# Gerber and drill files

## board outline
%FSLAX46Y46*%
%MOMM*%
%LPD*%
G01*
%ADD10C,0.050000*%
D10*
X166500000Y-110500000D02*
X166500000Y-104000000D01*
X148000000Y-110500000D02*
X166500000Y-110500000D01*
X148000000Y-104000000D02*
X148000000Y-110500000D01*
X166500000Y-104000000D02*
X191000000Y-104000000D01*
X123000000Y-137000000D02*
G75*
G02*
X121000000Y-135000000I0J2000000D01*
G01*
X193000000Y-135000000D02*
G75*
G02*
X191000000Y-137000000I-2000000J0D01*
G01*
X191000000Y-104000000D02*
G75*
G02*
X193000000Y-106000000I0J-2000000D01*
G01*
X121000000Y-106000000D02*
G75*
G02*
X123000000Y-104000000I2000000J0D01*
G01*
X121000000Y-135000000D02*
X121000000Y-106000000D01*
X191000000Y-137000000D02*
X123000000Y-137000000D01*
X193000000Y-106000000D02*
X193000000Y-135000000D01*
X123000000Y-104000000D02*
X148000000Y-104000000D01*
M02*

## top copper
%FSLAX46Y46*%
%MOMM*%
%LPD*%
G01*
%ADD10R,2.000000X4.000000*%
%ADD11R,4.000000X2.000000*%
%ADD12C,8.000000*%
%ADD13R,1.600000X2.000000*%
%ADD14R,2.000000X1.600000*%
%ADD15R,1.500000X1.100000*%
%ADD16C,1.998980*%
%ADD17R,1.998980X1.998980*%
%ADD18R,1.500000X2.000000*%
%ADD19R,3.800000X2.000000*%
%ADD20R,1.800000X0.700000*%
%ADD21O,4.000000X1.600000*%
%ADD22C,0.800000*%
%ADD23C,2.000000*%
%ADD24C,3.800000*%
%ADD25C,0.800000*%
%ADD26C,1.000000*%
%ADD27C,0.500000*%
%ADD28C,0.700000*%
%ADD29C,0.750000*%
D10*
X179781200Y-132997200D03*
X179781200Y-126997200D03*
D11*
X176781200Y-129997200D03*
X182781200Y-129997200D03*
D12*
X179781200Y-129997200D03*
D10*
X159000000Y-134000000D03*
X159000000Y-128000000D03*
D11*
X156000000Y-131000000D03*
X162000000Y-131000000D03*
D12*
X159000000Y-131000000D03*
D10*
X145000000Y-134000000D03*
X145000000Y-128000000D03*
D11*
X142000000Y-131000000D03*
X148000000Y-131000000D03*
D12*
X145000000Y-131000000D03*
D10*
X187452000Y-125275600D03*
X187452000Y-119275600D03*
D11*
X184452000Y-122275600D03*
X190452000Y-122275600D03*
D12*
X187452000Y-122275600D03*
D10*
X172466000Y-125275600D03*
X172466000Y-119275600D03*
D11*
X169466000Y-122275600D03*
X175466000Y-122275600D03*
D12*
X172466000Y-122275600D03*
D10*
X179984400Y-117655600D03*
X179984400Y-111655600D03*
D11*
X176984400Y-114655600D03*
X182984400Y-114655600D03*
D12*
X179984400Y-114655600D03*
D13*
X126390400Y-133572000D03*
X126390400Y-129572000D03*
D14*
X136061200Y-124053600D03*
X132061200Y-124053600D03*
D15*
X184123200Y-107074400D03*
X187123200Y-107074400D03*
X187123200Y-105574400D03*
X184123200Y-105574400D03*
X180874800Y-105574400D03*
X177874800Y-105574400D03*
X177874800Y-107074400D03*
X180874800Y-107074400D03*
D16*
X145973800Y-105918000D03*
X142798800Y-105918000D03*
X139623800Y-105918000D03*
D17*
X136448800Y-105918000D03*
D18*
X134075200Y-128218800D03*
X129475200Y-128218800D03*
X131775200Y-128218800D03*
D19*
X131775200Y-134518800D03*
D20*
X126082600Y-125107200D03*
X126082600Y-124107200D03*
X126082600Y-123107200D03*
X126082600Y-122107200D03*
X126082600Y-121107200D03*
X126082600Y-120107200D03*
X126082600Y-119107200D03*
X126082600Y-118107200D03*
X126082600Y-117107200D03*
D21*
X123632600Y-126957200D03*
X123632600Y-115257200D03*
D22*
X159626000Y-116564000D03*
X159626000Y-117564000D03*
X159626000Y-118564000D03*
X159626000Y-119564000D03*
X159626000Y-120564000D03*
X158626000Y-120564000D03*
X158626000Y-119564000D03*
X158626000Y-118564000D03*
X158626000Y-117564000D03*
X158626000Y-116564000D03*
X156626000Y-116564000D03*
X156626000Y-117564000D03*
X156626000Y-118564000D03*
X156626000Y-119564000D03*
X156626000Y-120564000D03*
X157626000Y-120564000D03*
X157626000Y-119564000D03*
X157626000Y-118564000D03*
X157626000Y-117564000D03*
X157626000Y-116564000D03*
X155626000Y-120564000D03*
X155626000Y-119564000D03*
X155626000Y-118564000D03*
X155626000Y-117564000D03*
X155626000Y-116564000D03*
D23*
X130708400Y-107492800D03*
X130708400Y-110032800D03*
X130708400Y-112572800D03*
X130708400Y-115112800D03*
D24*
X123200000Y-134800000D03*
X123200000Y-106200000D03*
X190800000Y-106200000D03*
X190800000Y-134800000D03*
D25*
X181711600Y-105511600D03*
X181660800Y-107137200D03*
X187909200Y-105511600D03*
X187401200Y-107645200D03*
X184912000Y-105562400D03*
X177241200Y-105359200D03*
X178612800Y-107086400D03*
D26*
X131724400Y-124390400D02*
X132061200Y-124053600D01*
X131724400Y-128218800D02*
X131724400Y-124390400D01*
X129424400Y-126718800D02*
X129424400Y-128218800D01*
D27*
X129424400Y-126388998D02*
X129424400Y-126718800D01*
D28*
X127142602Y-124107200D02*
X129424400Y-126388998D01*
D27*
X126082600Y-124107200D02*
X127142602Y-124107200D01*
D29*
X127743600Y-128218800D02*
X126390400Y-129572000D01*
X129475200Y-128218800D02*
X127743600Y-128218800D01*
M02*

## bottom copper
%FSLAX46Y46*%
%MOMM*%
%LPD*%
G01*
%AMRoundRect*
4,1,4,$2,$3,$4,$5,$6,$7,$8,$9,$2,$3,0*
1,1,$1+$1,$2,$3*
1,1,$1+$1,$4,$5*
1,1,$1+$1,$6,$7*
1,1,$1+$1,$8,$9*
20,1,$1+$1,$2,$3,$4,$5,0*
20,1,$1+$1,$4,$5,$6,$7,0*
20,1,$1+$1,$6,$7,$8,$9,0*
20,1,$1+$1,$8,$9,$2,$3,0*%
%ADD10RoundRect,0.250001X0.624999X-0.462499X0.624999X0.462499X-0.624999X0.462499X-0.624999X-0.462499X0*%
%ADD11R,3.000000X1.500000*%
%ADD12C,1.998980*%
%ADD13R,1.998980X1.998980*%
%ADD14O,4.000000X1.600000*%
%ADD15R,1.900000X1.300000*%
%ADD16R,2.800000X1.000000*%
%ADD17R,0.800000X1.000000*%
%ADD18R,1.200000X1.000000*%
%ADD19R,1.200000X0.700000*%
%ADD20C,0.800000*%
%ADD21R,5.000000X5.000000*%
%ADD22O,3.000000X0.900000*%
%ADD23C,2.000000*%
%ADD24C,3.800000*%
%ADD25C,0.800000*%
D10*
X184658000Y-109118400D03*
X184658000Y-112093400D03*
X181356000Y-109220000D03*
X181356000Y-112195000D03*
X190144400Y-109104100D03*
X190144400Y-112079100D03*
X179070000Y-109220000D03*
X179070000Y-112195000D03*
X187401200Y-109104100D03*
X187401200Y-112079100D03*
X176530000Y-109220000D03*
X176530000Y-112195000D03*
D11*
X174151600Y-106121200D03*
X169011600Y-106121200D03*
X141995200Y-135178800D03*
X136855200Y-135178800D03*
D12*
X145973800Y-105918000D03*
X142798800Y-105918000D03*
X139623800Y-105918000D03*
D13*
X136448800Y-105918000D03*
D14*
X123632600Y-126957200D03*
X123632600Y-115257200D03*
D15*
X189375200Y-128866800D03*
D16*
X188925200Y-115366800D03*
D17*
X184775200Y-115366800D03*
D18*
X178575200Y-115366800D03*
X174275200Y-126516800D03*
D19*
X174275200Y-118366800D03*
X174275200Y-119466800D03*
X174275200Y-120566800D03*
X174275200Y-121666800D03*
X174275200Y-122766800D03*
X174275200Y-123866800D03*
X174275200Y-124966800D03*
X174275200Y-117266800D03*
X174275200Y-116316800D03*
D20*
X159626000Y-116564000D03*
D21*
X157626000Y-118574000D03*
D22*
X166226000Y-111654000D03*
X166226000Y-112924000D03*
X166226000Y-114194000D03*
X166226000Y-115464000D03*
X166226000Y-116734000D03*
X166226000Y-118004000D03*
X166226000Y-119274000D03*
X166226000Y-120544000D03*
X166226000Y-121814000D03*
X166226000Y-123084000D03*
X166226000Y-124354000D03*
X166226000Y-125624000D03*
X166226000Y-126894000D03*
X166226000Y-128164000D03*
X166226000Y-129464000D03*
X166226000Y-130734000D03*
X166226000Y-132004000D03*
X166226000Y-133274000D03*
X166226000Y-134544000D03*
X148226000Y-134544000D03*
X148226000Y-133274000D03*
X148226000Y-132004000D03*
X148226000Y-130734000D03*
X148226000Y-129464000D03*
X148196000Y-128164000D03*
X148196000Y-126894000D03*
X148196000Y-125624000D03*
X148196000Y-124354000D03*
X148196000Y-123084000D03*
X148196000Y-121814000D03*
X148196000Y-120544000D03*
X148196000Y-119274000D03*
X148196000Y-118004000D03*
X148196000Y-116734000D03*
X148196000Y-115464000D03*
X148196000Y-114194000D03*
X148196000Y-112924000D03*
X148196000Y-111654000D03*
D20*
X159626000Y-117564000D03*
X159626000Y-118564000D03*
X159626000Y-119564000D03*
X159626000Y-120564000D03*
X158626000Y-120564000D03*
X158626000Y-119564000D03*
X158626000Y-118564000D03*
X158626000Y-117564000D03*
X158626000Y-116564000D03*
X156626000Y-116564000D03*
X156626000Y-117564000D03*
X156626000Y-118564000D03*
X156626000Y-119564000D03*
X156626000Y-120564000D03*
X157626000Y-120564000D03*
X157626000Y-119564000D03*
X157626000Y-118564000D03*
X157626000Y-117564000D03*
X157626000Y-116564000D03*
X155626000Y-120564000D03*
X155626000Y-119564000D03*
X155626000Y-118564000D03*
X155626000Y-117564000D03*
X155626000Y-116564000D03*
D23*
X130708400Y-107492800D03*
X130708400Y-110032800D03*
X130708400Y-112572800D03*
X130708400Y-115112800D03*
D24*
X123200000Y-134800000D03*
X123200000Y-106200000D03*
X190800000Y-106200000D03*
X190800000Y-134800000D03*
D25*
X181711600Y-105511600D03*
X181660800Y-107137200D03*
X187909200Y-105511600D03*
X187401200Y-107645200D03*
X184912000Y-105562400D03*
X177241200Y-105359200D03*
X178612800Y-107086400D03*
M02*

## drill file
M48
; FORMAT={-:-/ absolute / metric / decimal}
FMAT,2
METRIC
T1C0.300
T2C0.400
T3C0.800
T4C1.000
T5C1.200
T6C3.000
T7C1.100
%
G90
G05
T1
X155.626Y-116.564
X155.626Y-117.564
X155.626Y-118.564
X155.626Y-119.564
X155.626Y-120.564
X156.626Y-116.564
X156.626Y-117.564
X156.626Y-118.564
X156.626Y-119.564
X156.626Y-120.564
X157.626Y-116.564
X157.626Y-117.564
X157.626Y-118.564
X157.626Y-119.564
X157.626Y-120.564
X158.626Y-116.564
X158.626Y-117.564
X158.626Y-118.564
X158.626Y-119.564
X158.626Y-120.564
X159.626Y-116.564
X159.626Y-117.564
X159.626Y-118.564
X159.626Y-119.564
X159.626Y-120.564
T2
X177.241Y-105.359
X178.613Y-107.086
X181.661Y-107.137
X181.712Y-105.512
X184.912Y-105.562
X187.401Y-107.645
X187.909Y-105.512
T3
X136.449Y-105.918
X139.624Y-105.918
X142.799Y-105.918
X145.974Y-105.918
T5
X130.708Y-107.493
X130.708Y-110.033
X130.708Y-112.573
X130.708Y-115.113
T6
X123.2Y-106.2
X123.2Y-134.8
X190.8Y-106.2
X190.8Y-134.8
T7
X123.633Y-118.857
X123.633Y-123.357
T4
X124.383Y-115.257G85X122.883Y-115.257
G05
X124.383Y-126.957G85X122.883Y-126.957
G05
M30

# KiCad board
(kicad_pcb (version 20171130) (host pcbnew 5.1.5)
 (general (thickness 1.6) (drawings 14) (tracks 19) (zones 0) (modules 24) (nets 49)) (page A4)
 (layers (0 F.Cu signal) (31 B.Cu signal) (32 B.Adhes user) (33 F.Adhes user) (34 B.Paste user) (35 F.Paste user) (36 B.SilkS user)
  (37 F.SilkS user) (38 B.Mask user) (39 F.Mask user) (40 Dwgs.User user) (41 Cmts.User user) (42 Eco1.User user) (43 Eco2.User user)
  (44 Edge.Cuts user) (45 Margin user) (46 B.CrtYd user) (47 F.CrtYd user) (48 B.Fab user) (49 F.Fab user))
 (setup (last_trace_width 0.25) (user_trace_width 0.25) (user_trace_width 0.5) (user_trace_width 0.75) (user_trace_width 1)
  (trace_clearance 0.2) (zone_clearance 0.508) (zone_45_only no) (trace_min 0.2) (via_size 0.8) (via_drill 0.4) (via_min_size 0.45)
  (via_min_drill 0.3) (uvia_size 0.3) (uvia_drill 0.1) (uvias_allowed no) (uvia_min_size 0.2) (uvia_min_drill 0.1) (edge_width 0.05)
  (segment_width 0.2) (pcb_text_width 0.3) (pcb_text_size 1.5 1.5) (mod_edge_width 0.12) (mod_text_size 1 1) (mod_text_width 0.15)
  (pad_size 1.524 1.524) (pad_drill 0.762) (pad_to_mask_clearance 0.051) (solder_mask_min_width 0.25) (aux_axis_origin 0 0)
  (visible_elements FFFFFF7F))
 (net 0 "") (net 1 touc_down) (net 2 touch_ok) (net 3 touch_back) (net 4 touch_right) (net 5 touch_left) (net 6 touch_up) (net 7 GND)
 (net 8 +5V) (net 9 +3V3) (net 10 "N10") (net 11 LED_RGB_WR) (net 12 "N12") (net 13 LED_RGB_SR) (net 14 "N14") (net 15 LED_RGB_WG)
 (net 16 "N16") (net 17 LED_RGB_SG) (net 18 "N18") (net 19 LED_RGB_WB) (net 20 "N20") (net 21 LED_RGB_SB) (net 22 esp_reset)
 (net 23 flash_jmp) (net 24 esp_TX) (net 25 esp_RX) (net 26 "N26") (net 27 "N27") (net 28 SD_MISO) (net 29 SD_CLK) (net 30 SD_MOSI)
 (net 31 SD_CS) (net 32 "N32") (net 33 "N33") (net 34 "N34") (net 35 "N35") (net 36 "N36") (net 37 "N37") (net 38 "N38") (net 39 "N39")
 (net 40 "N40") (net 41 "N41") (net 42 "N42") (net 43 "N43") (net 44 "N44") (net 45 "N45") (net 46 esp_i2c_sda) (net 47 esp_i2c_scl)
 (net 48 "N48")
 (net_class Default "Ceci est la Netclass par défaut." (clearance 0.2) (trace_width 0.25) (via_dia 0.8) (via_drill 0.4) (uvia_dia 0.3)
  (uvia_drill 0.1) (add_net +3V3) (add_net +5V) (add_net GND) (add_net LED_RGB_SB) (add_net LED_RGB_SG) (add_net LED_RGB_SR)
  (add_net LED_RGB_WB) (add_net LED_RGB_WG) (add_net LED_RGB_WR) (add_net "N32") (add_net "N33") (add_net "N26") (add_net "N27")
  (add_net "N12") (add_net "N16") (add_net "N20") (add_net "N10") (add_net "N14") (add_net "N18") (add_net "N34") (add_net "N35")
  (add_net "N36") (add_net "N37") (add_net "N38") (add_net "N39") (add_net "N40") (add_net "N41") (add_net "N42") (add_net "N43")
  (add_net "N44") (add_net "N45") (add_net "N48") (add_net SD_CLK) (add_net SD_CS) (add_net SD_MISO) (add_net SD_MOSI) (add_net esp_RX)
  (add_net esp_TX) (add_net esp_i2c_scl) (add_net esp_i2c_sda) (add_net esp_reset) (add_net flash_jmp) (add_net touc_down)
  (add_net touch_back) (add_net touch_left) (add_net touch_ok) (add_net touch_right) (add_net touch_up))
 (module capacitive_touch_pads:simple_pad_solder (layer F.Cu) (at 179.7812 129.9972)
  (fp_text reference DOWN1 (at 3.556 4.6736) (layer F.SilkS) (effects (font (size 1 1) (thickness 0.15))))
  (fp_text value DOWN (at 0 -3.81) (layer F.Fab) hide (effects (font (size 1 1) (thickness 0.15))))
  (pad 1 smd rect (at 0 3 180) (size 2 4) (layers F.Cu F.Paste F.Mask) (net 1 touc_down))
  (pad 1 smd rect (at 0 -3 180) (size 2 4) (layers F.Cu F.Paste F.Mask) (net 1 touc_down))
  (pad 1 smd rect (at -3 0 90) (size 2 4) (layers F.Cu F.Paste F.Mask) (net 1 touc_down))
  (pad 1 smd rect (at 3 0 90) (size 2 4) (layers F.Cu F.Paste F.Mask) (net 1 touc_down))
  (pad 1 smd circle (at 0 0) (size 8 8) (layers F.Cu F.Paste F.Mask) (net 1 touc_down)))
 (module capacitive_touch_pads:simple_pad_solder (layer F.Cu) (at 159 131)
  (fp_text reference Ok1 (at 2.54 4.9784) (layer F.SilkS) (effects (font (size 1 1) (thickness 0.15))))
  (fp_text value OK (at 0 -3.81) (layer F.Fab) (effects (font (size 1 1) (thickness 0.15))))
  (pad 1 smd rect (at 0 3 180) (size 2 4) (layers F.Cu F.Paste F.Mask) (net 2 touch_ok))
  (pad 1 smd rect (at 0 -3 180) (size 2 4) (layers F.Cu F.Paste F.Mask) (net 2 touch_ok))
  (pad 1 smd rect (at -3 0 90) (size 2 4) (layers F.Cu F.Paste F.Mask) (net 2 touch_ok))
  (pad 1 smd rect (at 3 0 90) (size 2 4) (layers F.Cu F.Paste F.Mask) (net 2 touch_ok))
  (pad 1 smd circle (at 0 0) (size 8 8) (layers F.Cu F.Paste F.Mask) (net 2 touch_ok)))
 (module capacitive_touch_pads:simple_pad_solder (layer F.Cu) (at 145 131)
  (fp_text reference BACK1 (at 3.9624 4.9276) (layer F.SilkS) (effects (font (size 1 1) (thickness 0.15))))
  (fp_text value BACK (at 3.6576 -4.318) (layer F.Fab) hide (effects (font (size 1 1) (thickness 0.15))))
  (pad 1 smd rect (at 0 3 180) (size 2 4) (layers F.Cu F.Paste F.Mask) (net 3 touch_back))
  (pad 1 smd rect (at 0 -3 180) (size 2 4) (layers F.Cu F.Paste F.Mask) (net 3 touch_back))
  (pad 1 smd rect (at -3 0 90) (size 2 4) (layers F.Cu F.Paste F.Mask) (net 3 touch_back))
  (pad 1 smd rect (at 3 0 90) (size 2 4) (layers F.Cu F.Paste F.Mask) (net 3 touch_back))
  (pad 1 smd circle (at 0 0) (size 8 8) (layers F.Cu F.Paste F.Mask) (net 3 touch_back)))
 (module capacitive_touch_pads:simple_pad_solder (layer F.Cu) (at 187.452 122.2756)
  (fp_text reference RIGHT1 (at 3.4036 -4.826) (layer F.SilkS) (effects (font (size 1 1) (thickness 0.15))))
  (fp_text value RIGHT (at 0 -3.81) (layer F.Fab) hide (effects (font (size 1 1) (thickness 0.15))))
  (pad 1 smd rect (at 0 3 180) (size 2 4) (layers F.Cu F.Paste F.Mask) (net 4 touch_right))
  (pad 1 smd rect (at 0 -3 180) (size 2 4) (layers F.Cu F.Paste F.Mask) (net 4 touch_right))
  (pad 1 smd rect (at -3 0 90) (size 2 4) (layers F.Cu F.Paste F.Mask) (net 4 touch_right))
  (pad 1 smd rect (at 3 0 90) (size 2 4) (layers F.Cu F.Paste F.Mask) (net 4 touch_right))
  (pad 1 smd circle (at 0 0) (size 8 8) (layers F.Cu F.Paste F.Mask) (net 4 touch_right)))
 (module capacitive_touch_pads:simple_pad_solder (layer F.Cu) (at 172.466 122.2756)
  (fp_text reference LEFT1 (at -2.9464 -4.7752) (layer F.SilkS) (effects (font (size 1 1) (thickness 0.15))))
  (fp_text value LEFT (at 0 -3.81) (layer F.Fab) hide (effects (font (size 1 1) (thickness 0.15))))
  (pad 1 smd rect (at 0 3 180) (size 2 4) (layers F.Cu F.Paste F.Mask) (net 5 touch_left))
  (pad 1 smd rect (at 0 -3 180) (size 2 4) (layers F.Cu F.Paste F.Mask) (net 5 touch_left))
  (pad 1 smd rect (at -3 0 90) (size 2 4) (layers F.Cu F.Paste F.Mask) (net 5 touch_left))
  (pad 1 smd rect (at 3 0 90) (size 2 4) (layers F.Cu F.Paste F.Mask) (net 5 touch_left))
  (pad 1 smd circle (at 0 0) (size 8 8) (layers F.Cu F.Paste F.Mask) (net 5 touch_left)))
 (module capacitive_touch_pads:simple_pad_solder (layer F.Cu) (at 179.9844 114.6556)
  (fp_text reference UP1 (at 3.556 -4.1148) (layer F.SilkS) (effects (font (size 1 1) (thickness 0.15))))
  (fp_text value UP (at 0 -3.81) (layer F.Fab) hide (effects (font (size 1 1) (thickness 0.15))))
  (pad 1 smd rect (at 0 3 180) (size 2 4) (layers F.Cu F.Paste F.Mask) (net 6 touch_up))
  (pad 1 smd rect (at 0 -3 180) (size 2 4) (layers F.Cu F.Paste F.Mask) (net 6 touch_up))
  (pad 1 smd rect (at -3 0 90) (size 2 4) (layers F.Cu F.Paste F.Mask) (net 6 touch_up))
  (pad 1 smd rect (at 3 0 90) (size 2 4) (layers F.Cu F.Paste F.Mask) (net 6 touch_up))
  (pad 1 smd circle (at 0 0) (size 8 8) (layers F.Cu F.Paste F.Mask) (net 6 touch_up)))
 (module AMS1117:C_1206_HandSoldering (layer F.Cu) (at 126.3904 131.572 270)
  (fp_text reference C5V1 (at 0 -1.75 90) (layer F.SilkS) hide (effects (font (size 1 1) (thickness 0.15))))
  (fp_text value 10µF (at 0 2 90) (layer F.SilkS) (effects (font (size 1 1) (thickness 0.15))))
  (pad 2 smd rect (at 2 0 270) (size 2 1.6) (layers F.Cu F.Paste F.Mask) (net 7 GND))
  (pad 1 smd rect (at -2 0 270) (size 2 1.6) (layers F.Cu F.Paste F.Mask) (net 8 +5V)))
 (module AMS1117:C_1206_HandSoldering (layer F.Cu) (at 134.0612 124.0536)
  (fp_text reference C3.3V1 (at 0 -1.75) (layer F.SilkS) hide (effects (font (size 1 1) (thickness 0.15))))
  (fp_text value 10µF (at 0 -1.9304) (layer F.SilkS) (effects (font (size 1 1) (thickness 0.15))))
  (pad 2 smd rect (at 2 0) (size 2 1.6) (layers F.Cu F.Paste F.Mask) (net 7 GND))
  (pad 1 smd rect (at -2 0) (size 2 1.6) (layers F.Cu F.Paste F.Mask) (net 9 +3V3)))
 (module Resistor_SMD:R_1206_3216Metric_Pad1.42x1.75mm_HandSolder (layer B.Cu) (at 184.658 110.6059 90)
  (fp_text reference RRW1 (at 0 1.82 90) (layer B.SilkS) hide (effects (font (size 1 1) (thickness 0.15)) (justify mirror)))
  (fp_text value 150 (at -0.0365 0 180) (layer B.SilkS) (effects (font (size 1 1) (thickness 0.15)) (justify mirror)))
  (pad 2 smd roundrect (at 1.4875 0 90) (size 1.425 1.75) (layers B.Cu B.Paste B.Mask) (roundrect_rratio 0.175439) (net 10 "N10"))
  (pad 1 smd roundrect (at -1.4875 0 90) (size 1.425 1.75) (layers B.Cu B.Paste B.Mask) (roundrect_rratio 0.175439) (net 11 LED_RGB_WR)))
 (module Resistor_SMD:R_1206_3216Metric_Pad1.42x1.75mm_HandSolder (layer B.Cu) (at 181.356 110.7075 90)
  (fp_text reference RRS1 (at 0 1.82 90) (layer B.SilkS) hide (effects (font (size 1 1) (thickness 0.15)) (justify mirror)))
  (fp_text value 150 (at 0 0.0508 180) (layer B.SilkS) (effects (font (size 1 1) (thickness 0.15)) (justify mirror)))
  (pad 2 smd roundrect (at 1.4875 0 90) (size 1.425 1.75) (layers B.Cu B.Paste B.Mask) (roundrect_rratio 0.175439) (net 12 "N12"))
  (pad 1 smd roundrect (at -1.4875 0 90) (size 1.425 1.75) (layers B.Cu B.Paste B.Mask) (roundrect_rratio 0.175439) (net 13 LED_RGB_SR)))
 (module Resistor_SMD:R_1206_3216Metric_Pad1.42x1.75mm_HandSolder (layer B.Cu) (at 190.1444 110.5916 90)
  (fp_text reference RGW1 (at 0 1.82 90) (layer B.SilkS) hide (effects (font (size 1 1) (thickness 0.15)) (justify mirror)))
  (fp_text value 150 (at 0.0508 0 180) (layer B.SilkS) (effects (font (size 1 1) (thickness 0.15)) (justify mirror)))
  (pad 2 smd roundrect (at 1.4875 0 90) (size 1.425 1.75) (layers B.Cu B.Paste B.Mask) (roundrect_rratio 0.175439) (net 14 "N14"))
  (pad 1 smd roundrect (at -1.4875 0 90) (size 1.425 1.75) (layers B.Cu B.Paste B.Mask) (roundrect_rratio 0.175439) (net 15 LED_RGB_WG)))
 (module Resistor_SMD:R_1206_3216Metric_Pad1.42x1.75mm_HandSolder (layer B.Cu) (at 179.07 110.7075 90)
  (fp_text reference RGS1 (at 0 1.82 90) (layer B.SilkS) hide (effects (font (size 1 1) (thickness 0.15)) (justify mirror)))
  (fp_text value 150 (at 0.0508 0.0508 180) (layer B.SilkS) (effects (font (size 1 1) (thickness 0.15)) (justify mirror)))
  (pad 2 smd roundrect (at 1.4875 0 90) (size 1.425 1.75) (layers B.Cu B.Paste B.Mask) (roundrect_rratio 0.175439) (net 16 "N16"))
  (pad 1 smd roundrect (at -1.4875 0 90) (size 1.425 1.75) (layers B.Cu B.Paste B.Mask) (roundrect_rratio 0.175439) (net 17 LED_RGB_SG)))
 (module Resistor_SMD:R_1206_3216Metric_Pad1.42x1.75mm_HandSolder (layer B.Cu) (at 187.4012 110.5916 90)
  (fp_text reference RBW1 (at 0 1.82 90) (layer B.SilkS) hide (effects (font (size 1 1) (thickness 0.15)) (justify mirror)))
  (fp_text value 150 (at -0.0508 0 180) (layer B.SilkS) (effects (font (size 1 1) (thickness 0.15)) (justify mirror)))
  (pad 2 smd roundrect (at 1.4875 0 90) (size 1.425 1.75) (layers B.Cu B.Paste B.Mask) (roundrect_rratio 0.175439) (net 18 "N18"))
  (pad 1 smd roundrect (at -1.4875 0 90) (size 1.425 1.75) (layers B.Cu B.Paste B.Mask) (roundrect_rratio 0.175439) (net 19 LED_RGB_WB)))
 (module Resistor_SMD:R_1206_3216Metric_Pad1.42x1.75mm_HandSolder (layer B.Cu) (at 176.53 110.7075 90)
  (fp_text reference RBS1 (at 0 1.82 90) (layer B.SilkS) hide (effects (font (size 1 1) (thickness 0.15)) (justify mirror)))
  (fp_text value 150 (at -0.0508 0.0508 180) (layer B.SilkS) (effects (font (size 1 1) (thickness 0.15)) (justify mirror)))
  (pad 2 smd roundrect (at 1.4875 0 90) (size 1.425 1.75) (layers B.Cu B.Paste B.Mask) (roundrect_rratio 0.175439) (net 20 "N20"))
  (pad 1 smd roundrect (at -1.4875 0 90) (size 1.425 1.75) (layers B.Cu B.Paste B.Mask) (roundrect_rratio 0.175439) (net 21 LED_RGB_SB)))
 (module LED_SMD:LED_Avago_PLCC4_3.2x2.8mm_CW (layer F.Cu) (at 185.6232 106.3244)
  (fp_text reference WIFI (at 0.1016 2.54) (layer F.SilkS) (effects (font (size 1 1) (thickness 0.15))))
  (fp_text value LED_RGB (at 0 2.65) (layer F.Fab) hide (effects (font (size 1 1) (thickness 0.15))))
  (pad 4 smd rect (at -1.5 0.75) (size 1.5 1.1) (layers F.Cu F.Paste F.Mask) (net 9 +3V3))
  (pad 3 smd rect (at 1.5 0.75) (size 1.5 1.1) (layers F.Cu F.Paste F.Mask) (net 18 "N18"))
  (pad 2 smd rect (at 1.5 -0.75) (size 1.5 1.1) (layers F.Cu F.Paste F.Mask) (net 14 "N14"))
  (pad 1 smd rect (at -1.5 -0.75) (size 1.5 1.1) (layers F.Cu F.Paste F.Mask) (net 10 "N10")))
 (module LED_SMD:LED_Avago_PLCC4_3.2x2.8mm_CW (layer F.Cu) (at 179.3748 106.3244 180)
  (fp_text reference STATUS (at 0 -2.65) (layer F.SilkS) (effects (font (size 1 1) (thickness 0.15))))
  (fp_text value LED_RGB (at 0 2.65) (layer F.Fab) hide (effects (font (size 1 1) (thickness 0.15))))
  (pad 4 smd rect (at -1.5 0.75 180) (size 1.5 1.1) (layers F.Cu F.Paste F.Mask) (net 9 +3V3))
  (pad 3 smd rect (at 1.5 0.75 180) (size 1.5 1.1) (layers F.Cu F.Paste F.Mask) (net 20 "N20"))
  (pad 2 smd rect (at 1.5 -0.75 180) (size 1.5 1.1) (layers F.Cu F.Paste F.Mask) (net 16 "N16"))
  (pad 1 smd rect (at -1.5 -0.75 180) (size 1.5 1.1) (layers F.Cu F.Paste F.Mask) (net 12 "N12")))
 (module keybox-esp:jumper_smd (layer B.Cu) (at 171.5516 106.1212 270)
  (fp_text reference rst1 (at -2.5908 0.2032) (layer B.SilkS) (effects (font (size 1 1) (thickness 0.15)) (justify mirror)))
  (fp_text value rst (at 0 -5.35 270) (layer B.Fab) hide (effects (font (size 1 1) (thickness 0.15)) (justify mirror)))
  (pad 2 smd rect (at 0 -2.6 270) (size 1.5 3) (layers B.Cu B.Paste B.Mask) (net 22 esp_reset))
  (pad 1 smd rect (at 0 2.54 270) (size 1.5 3) (layers B.Cu B.Paste B.Mask) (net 7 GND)))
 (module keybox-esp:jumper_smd (layer B.Cu) (at 139.3952 135.1788 270)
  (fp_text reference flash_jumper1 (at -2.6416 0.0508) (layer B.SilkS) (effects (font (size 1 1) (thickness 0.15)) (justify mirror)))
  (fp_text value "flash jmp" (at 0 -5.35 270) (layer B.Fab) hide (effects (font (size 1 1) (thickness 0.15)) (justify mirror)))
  (pad 2 smd rect (at 0 -2.6 270) (size 1.5 3) (layers B.Cu B.Paste B.Mask) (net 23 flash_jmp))
  (pad 1 smd rect (at 0 2.54 270) (size 1.5 3) (layers B.Cu B.Paste B.Mask) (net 7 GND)))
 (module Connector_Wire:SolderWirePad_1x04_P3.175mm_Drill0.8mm (layer B.Cu) (at 136.4488 105.918)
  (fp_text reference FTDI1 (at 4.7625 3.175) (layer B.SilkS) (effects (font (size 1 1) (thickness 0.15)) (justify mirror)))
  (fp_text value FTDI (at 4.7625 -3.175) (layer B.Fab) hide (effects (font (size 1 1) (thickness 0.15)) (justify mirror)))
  (pad 4 thru_hole circle (at 9.525 0) (size 1.99898 1.99898) (drill 0.8001) (layers *.Cu *.Mask) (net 7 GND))
  (pad 3 thru_hole circle (at 6.35 0) (size 1.99898 1.99898) (drill 0.8001) (layers *.Cu *.Mask) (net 9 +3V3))
  (pad 2 thru_hole circle (at 3.175 0) (size 1.99898 1.99898) (drill 0.8001) (layers *.Cu *.Mask) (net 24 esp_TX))
  (pad 1 thru_hole rect (at 0 0) (size 1.99898 1.99898) (drill 0.8001) (layers *.Cu *.Mask) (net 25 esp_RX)))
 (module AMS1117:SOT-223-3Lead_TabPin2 (layer F.Cu) (at 131.7752 131.3688 270)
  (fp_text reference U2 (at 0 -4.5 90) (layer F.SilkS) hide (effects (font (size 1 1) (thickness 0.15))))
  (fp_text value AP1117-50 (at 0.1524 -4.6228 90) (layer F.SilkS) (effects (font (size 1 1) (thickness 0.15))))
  (pad 1 smd rect (at -3.15 -2.3 270) (size 2 1.5) (layers F.Cu F.Paste F.Mask) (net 7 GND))
  (pad 3 smd rect (at -3.15 2.3 270) (size 2 1.5) (layers F.Cu F.Paste F.Mask) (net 8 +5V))
  (pad 2 smd rect (at -3.15 0 270) (size 2 1.5) (layers F.Cu F.Paste F.Mask) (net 9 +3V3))
  (pad 2 smd rect (at 3.15 0 270) (size 2 3.8) (layers F.Cu F.Paste F.Mask) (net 9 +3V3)))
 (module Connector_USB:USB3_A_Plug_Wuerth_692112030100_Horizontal (layer F.Cu) (at 124.3076 121.1072 180)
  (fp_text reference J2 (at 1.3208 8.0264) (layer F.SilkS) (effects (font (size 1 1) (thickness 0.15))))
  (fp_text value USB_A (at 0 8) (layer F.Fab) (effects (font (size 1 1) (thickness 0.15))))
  (pad "" np_thru_hole circle (at 0.675 -2.25 270) (size 1.1 1.1) (drill 1.1) (layers *.Cu *.Mask))
  (pad "" np_thru_hole circle (at 0.675 2.25 270) (size 1.1 1.1) (drill 1.1) (layers *.Cu *.Mask))
  (pad 9 smd rect (at -1.775 -4 180) (size 1.8 0.7) (layers F.Cu F.Paste F.Mask))
  (pad 1 smd rect (at -1.775 -3 270) (size 0.7 1.8) (layers F.Cu F.Paste F.Mask) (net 8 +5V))
  (pad 8 smd rect (at -1.775 -2 270) (size 0.7 1.8) (layers F.Cu F.Paste F.Mask))
  (pad 2 smd rect (at -1.775 -1 270) (size 0.7 1.8) (layers F.Cu F.Paste F.Mask) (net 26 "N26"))
  (pad 7 smd rect (at -1.775 0 270) (size 0.7 1.8) (layers F.Cu F.Paste F.Mask))
  (pad 3 smd rect (at -1.775 1 270) (size 0.7 1.8) (layers F.Cu F.Paste F.Mask) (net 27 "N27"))
  (pad 6 smd rect (at -1.775 2 270) (size 0.7 1.8) (layers F.Cu F.Paste F.Mask))
  (pad 4 smd rect (at -1.775 3 270) (size 0.7 1.8) (layers F.Cu F.Paste F.Mask) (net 7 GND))
  (pad 5 smd rect (at -1.775 4 270) (size 0.7 1.8) (layers F.Cu F.Paste F.Mask) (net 7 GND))
  (pad 10 thru_hole oval (at 0.675 -5.85 270) (size 1.6 4) (drill oval 1 2.5) (layers *.Cu *.Mask))
  (pad 10 thru_hole oval (at 0.675 5.85 270) (size 1.6 4) (drill oval 1 2.5) (layers *.Cu *.Mask)))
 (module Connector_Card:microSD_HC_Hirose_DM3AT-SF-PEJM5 (layer B.Cu) (at 182.0002 122.1918 270)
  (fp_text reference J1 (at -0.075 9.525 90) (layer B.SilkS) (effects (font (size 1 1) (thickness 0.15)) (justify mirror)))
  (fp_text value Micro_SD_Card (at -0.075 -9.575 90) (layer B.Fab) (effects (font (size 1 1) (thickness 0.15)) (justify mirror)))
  (pad 11 smd rect (at 6.675 -7.375 270) (size 1.3 1.9) (layers B.Cu B.Paste B.Mask))
  (pad 11 smd rect (at -6.825 -6.925 270) (size 1 2.8) (layers B.Cu B.Paste B.Mask))
  (pad 10 smd rect (at -6.825 -2.775 270) (size 1 0.8) (layers B.Cu B.Paste B.Mask))
  (pad 11 smd rect (at -6.825 3.425 270) (size 1 1.2) (layers B.Cu B.Paste B.Mask))
  (pad 11 smd rect (at 4.325 7.725 270) (size 1 1.2) (layers B.Cu B.Paste B.Mask))
  (pad 7 smd rect (at -3.825 7.725 270) (size 0.7 1.2) (layers B.Cu B.Paste B.Mask) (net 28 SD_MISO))
  (pad 6 smd rect (at -2.725 7.725 270) (size 0.7 1.2) (layers B.Cu B.Paste B.Mask) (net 7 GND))
  (pad 5 smd rect (at -1.625 7.725 270) (size 0.7 1.2) (layers B.Cu B.Paste B.Mask) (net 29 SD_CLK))
  (pad 4 smd rect (at -0.525 7.725 270) (size 0.7 1.2) (layers B.Cu B.Paste B.Mask) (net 9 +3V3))
  (pad 3 smd rect (at 0.575 7.725 270) (size 0.7 1.2) (layers B.Cu B.Paste B.Mask) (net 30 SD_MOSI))
  (pad 2 smd rect (at 1.675 7.725 270) (size 0.7 1.2) (layers B.Cu B.Paste B.Mask) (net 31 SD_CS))
  (pad 1 smd rect (at 2.775 7.725 270) (size 0.7 1.2) (layers B.Cu B.Paste B.Mask) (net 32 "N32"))
  (pad 8 smd rect (at -4.925 7.725 270) (size 0.7 1.2) (layers B.Cu B.Paste B.Mask) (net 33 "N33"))
  (pad 9 smd rect (at -5.875 7.725 270) (size 0.7 1.2) (layers B.Cu B.Paste B.Mask) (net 7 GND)))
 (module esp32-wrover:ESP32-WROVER (layer B.Cu) (at 157.226 110.744 180)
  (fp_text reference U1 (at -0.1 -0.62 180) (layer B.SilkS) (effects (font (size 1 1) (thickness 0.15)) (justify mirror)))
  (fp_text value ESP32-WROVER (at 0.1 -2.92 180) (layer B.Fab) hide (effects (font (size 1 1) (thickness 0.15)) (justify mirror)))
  (pad 39 thru_hole circle (at -2.4 -5.82 180) (size 0.8 0.8) (drill 0.3) (layers *.Cu *.Mask) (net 7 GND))
  (pad 39 smd rect (at -0.4 -7.83 180) (size 5 5) (layers B.Cu B.Paste B.Mask) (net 7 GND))
  (pad 1 smd oval (at -9 -0.91 180) (size 3 0.9) (layers B.Cu B.Paste B.Mask) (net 7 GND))
  (pad 2 smd oval (at -9 -2.18 180) (size 3 0.9) (layers B.Cu B.Paste B.Mask) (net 9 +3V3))
  (pad 3 smd oval (at -9 -3.45 180) (size 3 0.9) (layers B.Cu B.Paste B.Mask) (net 22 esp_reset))
  (pad 4 smd oval (at -9 -4.72 180) (size 3 0.9) (layers B.Cu B.Paste B.Mask) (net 19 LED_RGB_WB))
  (pad 5 smd oval (at -9 -5.99 180) (size 3 0.9) (layers B.Cu B.Paste B.Mask) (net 15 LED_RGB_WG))
  (pad 6 smd oval (at -9 -7.26 180) (size 3 0.9) (layers B.Cu B.Paste B.Mask) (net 11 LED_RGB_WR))
  (pad 7 smd oval (at -9 -8.53 180) (size 3 0.9) (layers B.Cu B.Paste B.Mask) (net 13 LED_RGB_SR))
  (pad 8 smd oval (at -9 -9.8 180) (size 3 0.9) (layers B.Cu B.Paste B.Mask) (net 17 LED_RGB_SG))
  (pad 9 smd oval (at -9 -11.07 180) (size 3 0.9) (layers B.Cu B.Paste B.Mask) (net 21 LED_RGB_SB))
  (pad 10 smd oval (at -9 -12.34 180) (size 3 0.9) (layers B.Cu B.Paste B.Mask) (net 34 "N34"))
  (pad 11 smd oval (at -9 -13.61 180) (size 3 0.9) (layers B.Cu B.Paste B.Mask) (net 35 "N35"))
  (pad 12 smd oval (at -9 -14.88 180) (size 3 0.9) (layers B.Cu B.Paste B.Mask) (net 1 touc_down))
  (pad 13 smd oval (at -9 -16.15 180) (size 3 0.9) (layers B.Cu B.Paste B.Mask) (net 6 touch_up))
  (pad 14 smd oval (at -9 -17.42 180) (size 3 0.9) (layers B.Cu B.Paste B.Mask) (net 4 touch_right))
  (pad 15 smd oval (at -9 -18.72 180) (size 3 0.9) (layers B.Cu B.Paste B.Mask) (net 7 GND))
  (pad 16 smd oval (at -9 -19.99 180) (size 3 0.9) (layers B.Cu B.Paste B.Mask) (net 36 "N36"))
  (pad 17 smd oval (at -9 -21.26 180) (size 3 0.9) (layers B.Cu B.Paste B.Mask) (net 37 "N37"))
  (pad 18 smd oval (at -9 -22.53 180) (size 3 0.9) (layers B.Cu B.Paste B.Mask) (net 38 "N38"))
  (pad 19 smd oval (at -9 -23.8 180) (size 3 0.9) (layers B.Cu B.Paste B.Mask) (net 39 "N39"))
  (pad 20 smd oval (at 9 -23.8 180) (size 3 0.9) (layers B.Cu B.Paste B.Mask) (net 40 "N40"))
  (pad 21 smd oval (at 9 -22.53 180) (size 3 0.9) (layers B.Cu B.Paste B.Mask) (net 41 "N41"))
  (pad 22 smd oval (at 9 -21.26 180) (size 3 0.9) (layers B.Cu B.Paste B.Mask) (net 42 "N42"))
  (pad 23 smd oval (at 9 -19.99 180) (size 3 0.9) (layers B.Cu B.Paste B.Mask) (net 5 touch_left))
  (pad 24 smd oval (at 9 -18.72 180) (size 3 0.9) (layers B.Cu B.Paste B.Mask) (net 2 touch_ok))
  (pad 25 smd oval (at 9.03 -17.42 180) (size 3 0.9) (layers B.Cu B.Paste B.Mask) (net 23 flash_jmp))
  (pad 26 smd oval (at 9.03 -16.15 180) (size 3 0.9) (layers B.Cu B.Paste B.Mask) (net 3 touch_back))
  (pad 27 smd oval (at 9.03 -14.88 180) (size 3 0.9) (layers B.Cu B.Paste B.Mask) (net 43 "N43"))
  (pad 28 smd oval (at 9.03 -13.61 180) (size 3 0.9) (layers B.Cu B.Paste B.Mask) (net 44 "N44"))
  (pad 29 smd oval (at 9.03 -12.34 180) (size 3 0.9) (layers B.Cu B.Paste B.Mask) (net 31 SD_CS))
  (pad 30 smd oval (at 9.03 -11.07 180) (size 3 0.9) (layers B.Cu B.Paste B.Mask) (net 29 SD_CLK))
  (pad 31 smd oval (at 9.03 -9.8 180) (size 3 0.9) (layers B.Cu B.Paste B.Mask) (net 28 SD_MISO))
  (pad 32 smd oval (at 9.03 -8.53 180) (size 3 0.9) (layers B.Cu B.Paste B.Mask) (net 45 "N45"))
  (pad 33 smd oval (at 9.03 -7.26 180) (size 3 0.9) (layers B.Cu B.Paste B.Mask) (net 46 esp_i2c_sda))
  (pad 34 smd oval (at 9.03 -5.99 180) (size 3 0.9) (layers B.Cu B.Paste B.Mask) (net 25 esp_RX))
  (pad 35 smd oval (at 9.03 -4.72 180) (size 3 0.9) (layers B.Cu B.Paste B.Mask) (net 24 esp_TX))
  (pad 36 smd oval (at 9.03 -3.45 180) (size 3 0.9) (layers B.Cu B.Paste B.Mask) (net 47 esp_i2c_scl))
  (pad 37 smd oval (at 9.03 -2.18 180) (size 3 0.9) (layers B.Cu B.Paste B.Mask) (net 30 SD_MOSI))
  (pad 38 smd oval (at 9.03 -0.91 180) (size 3 0.9) (layers B.Cu B.Paste B.Mask) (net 7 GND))
  (pad 39 thru_hole circle (at -2.4 -6.82 180) (size 0.8 0.8) (drill 0.3) (layers *.Cu *.Mask) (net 7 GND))
  (pad 39 thru_hole circle (at -2.4 -7.82 180) (size 0.8 0.8) (drill 0.3) (layers *.Cu *.Mask) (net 7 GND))
  (pad 39 thru_hole circle (at -2.4 -8.82 180) (size 0.8 0.8) (drill 0.3) (layers *.Cu *.Mask) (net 7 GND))
  (pad 39 thru_hole circle (at -2.4 -9.82 180) (size 0.8 0.8) (drill 0.3) (layers *.Cu *.Mask) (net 7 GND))
  (pad 39 thru_hole circle (at -1.4 -9.82 180) (size 0.8 0.8) (drill 0.3) (layers *.Cu *.Mask) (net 7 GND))
  (pad 39 thru_hole circle (at -1.4 -8.82 180) (size 0.8 0.8) (drill 0.3) (layers *.Cu *.Mask) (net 7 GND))
  (pad 39 thru_hole circle (at -1.4 -7.82 180) (size 0.8 0.8) (drill 0.3) (layers *.Cu *.Mask) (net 7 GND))
  (pad 39 thru_hole circle (at -1.4 -6.82 180) (size 0.8 0.8) (drill 0.3) (layers *.Cu *.Mask) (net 7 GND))
  (pad 39 thru_hole circle (at -1.4 -5.82 180) (size 0.8 0.8) (drill 0.3) (layers *.Cu *.Mask) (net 7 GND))
  (pad 39 thru_hole circle (at 0.6 -5.82 180) (size 0.8 0.8) (drill 0.3) (layers *.Cu *.Mask) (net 7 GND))
  (pad 39 thru_hole circle (at 0.6 -6.82 180) (size 0.8 0.8) (drill 0.3) (layers *.Cu *.Mask) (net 7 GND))
  (pad 39 thru_hole circle (at 0.6 -7.82 180) (size 0.8 0.8) (drill 0.3) (layers *.Cu *.Mask) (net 7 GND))
  (pad 39 thru_hole circle (at 0.6 -8.82 180) (size 0.8 0.8) (drill 0.3) (layers *.Cu *.Mask) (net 7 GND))
  (pad 39 thru_hole circle (at 0.6 -9.82 180) (size 0.8 0.8) (drill 0.3) (layers *.Cu *.Mask) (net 7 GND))
  (pad 39 thru_hole circle (at -0.4 -9.82 180) (size 0.8 0.8) (drill 0.3) (layers *.Cu *.Mask) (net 7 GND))
  (pad 39 thru_hole circle (at -0.4 -8.82 180) (size 0.8 0.8) (drill 0.3) (layers *.Cu *.Mask) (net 7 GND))
  (pad 39 thru_hole circle (at -0.4 -7.82 180) (size 0.8 0.8) (drill 0.3) (layers *.Cu *.Mask) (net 7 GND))
  (pad 39 thru_hole circle (at -0.4 -6.82 180) (size 0.8 0.8) (drill 0.3) (layers *.Cu *.Mask) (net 7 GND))
  (pad 39 thru_hole circle (at -0.4 -5.82 180) (size 0.8 0.8) (drill 0.3) (layers *.Cu *.Mask) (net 7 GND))
  (pad 39 thru_hole circle (at 1.6 -9.82 180) (size 0.8 0.8) (drill 0.3) (layers *.Cu *.Mask) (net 7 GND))
  (pad 39 thru_hole circle (at 1.6 -8.82 180) (size 0.8 0.8) (drill 0.3) (layers *.Cu *.Mask) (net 7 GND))
  (pad 39 thru_hole circle (at 1.6 -7.82 180) (size 0.8 0.8) (drill 0.3) (layers *.Cu *.Mask) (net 7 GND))
  (pad 39 thru_hole circle (at 1.6 -6.82 180) (size 0.8 0.8) (drill 0.3) (layers *.Cu *.Mask) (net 7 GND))
  (pad 39 thru_hole circle (at 1.6 -5.82 180) (size 0.8 0.8) (drill 0.3) (layers *.Cu *.Mask) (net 7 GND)))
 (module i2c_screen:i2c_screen (layer F.Cu) (at 130.7084 115.1128)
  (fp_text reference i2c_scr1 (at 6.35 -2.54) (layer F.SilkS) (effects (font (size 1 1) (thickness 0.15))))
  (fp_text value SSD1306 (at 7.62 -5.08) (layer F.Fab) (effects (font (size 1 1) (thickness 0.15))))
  (pad SDA thru_hole circle (at 0 -7.62) (size 2 2) (drill 1.2) (layers *.Cu *.Mask) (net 46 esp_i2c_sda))
  (pad SCL thru_hole circle (at 0 -5.08) (size 2 2) (drill 1.2) (layers *.Cu *.Mask) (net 47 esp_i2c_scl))
  (pad VCC thru_hole circle (at 0 -2.54) (size 2 2) (drill 1.2) (layers *.Cu *.Mask) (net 9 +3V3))
  (pad GND thru_hole circle (at 0 0) (size 2 2) (drill 1.2) (layers *.Cu *.Mask) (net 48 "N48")))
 (gr_line (start 166.5 110.5) (end 166.5 104) (layer Edge.Cuts) (width 0.05))
 (gr_line (start 148 110.5) (end 166.5 110.5) (layer Edge.Cuts) (width 0.05))
 (gr_line (start 148 104) (end 148 110.5) (layer Edge.Cuts) (width 0.05))
 (gr_line (start 166.5 104) (end 191 104) (layer Edge.Cuts) (width 0.05))
 (gr_arc (start 123 135) (end 121 135) (angle -90) (layer Edge.Cuts) (width 0.05))
 (gr_arc (start 191 135) (end 191 137) (angle -90) (layer Edge.Cuts) (width 0.05))
 (gr_arc (start 191 106) (end 193 106) (angle -90) (layer Edge.Cuts) (width 0.05))
 (gr_arc (start 123 106) (end 123 104) (angle -90) (layer Edge.Cuts) (width 0.05))
 (gr_line (start 121 135) (end 121 106) (layer Edge.Cuts) (width 0.05))
 (gr_line (start 191 137) (end 123 137) (layer Edge.Cuts) (width 0.05))
 (gr_line (start 193 106) (end 193 135) (layer Edge.Cuts) (width 0.05))
 (gr_line (start 123 104) (end 148 104) (layer Edge.Cuts) (width 0.05))
 (via (at 123.2 134.8) (size 3.8) (drill 3) (layers F.Cu B.Cu) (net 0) (status 40000))
 (via (at 123.2 106.2) (size 3.8) (drill 3) (layers F.Cu B.Cu) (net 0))
 (via (at 190.8 106.2) (size 3.8) (drill 3) (layers F.Cu B.Cu) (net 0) (status 40000))
 (via (at 190.8 134.8) (size 3.8) (drill 3) (layers F.Cu B.Cu) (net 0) (status 40000))
 (via (at 181.7116 105.5116) (size 0.8) (drill 0.4) (layers F.Cu B.Cu) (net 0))
 (via (at 181.6608 107.1372) (size 0.8) (drill 0.4) (layers F.Cu B.Cu) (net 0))
 (via (at 187.9092 105.5116) (size 0.8) (drill 0.4) (layers F.Cu B.Cu) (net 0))
 (via (at 187.4012 107.6452) (size 0.8) (drill 0.4) (layers F.Cu B.Cu) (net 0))
 (via (at 184.912 105.5624) (size 0.8) (drill 0.4) (layers F.Cu B.Cu) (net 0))
 (segment (start 131.7244 124.3904) (end 132.0612 124.0536) (width 1) (layer F.Cu) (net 9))
 (segment (start 131.7244 128.2188) (end 131.7244 124.3904) (width 1) (layer F.Cu) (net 9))
 (segment (start 129.4244 126.7188) (end 129.4244 128.2188) (width 1) (layer F.Cu) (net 8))
 (segment (start 129.4244 126.388998) (end 129.4244 126.7188) (width 0.5) (layer F.Cu) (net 8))
 (segment (start 127.142602 124.1072) (end 129.4244 126.388998) (width 0.7) (layer F.Cu) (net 8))
 (segment (start 126.0826 124.1072) (end 127.142602 124.1072) (width 0.5) (layer F.Cu) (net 8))
 (segment (start 127.7436 128.2188) (end 126.3904 129.572) (width 0.75) (layer F.Cu) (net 8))
 (segment (start 129.4752 128.2188) (end 127.7436 128.2188) (width 0.75) (layer F.Cu) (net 8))
 (via (at 177.2412 105.3592) (size 0.8) (drill 0.4) (layers F.Cu B.Cu) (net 20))
 (via (at 178.6128 107.0864) (size 0.8) (drill 0.4) (layers F.Cu B.Cu) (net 16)))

